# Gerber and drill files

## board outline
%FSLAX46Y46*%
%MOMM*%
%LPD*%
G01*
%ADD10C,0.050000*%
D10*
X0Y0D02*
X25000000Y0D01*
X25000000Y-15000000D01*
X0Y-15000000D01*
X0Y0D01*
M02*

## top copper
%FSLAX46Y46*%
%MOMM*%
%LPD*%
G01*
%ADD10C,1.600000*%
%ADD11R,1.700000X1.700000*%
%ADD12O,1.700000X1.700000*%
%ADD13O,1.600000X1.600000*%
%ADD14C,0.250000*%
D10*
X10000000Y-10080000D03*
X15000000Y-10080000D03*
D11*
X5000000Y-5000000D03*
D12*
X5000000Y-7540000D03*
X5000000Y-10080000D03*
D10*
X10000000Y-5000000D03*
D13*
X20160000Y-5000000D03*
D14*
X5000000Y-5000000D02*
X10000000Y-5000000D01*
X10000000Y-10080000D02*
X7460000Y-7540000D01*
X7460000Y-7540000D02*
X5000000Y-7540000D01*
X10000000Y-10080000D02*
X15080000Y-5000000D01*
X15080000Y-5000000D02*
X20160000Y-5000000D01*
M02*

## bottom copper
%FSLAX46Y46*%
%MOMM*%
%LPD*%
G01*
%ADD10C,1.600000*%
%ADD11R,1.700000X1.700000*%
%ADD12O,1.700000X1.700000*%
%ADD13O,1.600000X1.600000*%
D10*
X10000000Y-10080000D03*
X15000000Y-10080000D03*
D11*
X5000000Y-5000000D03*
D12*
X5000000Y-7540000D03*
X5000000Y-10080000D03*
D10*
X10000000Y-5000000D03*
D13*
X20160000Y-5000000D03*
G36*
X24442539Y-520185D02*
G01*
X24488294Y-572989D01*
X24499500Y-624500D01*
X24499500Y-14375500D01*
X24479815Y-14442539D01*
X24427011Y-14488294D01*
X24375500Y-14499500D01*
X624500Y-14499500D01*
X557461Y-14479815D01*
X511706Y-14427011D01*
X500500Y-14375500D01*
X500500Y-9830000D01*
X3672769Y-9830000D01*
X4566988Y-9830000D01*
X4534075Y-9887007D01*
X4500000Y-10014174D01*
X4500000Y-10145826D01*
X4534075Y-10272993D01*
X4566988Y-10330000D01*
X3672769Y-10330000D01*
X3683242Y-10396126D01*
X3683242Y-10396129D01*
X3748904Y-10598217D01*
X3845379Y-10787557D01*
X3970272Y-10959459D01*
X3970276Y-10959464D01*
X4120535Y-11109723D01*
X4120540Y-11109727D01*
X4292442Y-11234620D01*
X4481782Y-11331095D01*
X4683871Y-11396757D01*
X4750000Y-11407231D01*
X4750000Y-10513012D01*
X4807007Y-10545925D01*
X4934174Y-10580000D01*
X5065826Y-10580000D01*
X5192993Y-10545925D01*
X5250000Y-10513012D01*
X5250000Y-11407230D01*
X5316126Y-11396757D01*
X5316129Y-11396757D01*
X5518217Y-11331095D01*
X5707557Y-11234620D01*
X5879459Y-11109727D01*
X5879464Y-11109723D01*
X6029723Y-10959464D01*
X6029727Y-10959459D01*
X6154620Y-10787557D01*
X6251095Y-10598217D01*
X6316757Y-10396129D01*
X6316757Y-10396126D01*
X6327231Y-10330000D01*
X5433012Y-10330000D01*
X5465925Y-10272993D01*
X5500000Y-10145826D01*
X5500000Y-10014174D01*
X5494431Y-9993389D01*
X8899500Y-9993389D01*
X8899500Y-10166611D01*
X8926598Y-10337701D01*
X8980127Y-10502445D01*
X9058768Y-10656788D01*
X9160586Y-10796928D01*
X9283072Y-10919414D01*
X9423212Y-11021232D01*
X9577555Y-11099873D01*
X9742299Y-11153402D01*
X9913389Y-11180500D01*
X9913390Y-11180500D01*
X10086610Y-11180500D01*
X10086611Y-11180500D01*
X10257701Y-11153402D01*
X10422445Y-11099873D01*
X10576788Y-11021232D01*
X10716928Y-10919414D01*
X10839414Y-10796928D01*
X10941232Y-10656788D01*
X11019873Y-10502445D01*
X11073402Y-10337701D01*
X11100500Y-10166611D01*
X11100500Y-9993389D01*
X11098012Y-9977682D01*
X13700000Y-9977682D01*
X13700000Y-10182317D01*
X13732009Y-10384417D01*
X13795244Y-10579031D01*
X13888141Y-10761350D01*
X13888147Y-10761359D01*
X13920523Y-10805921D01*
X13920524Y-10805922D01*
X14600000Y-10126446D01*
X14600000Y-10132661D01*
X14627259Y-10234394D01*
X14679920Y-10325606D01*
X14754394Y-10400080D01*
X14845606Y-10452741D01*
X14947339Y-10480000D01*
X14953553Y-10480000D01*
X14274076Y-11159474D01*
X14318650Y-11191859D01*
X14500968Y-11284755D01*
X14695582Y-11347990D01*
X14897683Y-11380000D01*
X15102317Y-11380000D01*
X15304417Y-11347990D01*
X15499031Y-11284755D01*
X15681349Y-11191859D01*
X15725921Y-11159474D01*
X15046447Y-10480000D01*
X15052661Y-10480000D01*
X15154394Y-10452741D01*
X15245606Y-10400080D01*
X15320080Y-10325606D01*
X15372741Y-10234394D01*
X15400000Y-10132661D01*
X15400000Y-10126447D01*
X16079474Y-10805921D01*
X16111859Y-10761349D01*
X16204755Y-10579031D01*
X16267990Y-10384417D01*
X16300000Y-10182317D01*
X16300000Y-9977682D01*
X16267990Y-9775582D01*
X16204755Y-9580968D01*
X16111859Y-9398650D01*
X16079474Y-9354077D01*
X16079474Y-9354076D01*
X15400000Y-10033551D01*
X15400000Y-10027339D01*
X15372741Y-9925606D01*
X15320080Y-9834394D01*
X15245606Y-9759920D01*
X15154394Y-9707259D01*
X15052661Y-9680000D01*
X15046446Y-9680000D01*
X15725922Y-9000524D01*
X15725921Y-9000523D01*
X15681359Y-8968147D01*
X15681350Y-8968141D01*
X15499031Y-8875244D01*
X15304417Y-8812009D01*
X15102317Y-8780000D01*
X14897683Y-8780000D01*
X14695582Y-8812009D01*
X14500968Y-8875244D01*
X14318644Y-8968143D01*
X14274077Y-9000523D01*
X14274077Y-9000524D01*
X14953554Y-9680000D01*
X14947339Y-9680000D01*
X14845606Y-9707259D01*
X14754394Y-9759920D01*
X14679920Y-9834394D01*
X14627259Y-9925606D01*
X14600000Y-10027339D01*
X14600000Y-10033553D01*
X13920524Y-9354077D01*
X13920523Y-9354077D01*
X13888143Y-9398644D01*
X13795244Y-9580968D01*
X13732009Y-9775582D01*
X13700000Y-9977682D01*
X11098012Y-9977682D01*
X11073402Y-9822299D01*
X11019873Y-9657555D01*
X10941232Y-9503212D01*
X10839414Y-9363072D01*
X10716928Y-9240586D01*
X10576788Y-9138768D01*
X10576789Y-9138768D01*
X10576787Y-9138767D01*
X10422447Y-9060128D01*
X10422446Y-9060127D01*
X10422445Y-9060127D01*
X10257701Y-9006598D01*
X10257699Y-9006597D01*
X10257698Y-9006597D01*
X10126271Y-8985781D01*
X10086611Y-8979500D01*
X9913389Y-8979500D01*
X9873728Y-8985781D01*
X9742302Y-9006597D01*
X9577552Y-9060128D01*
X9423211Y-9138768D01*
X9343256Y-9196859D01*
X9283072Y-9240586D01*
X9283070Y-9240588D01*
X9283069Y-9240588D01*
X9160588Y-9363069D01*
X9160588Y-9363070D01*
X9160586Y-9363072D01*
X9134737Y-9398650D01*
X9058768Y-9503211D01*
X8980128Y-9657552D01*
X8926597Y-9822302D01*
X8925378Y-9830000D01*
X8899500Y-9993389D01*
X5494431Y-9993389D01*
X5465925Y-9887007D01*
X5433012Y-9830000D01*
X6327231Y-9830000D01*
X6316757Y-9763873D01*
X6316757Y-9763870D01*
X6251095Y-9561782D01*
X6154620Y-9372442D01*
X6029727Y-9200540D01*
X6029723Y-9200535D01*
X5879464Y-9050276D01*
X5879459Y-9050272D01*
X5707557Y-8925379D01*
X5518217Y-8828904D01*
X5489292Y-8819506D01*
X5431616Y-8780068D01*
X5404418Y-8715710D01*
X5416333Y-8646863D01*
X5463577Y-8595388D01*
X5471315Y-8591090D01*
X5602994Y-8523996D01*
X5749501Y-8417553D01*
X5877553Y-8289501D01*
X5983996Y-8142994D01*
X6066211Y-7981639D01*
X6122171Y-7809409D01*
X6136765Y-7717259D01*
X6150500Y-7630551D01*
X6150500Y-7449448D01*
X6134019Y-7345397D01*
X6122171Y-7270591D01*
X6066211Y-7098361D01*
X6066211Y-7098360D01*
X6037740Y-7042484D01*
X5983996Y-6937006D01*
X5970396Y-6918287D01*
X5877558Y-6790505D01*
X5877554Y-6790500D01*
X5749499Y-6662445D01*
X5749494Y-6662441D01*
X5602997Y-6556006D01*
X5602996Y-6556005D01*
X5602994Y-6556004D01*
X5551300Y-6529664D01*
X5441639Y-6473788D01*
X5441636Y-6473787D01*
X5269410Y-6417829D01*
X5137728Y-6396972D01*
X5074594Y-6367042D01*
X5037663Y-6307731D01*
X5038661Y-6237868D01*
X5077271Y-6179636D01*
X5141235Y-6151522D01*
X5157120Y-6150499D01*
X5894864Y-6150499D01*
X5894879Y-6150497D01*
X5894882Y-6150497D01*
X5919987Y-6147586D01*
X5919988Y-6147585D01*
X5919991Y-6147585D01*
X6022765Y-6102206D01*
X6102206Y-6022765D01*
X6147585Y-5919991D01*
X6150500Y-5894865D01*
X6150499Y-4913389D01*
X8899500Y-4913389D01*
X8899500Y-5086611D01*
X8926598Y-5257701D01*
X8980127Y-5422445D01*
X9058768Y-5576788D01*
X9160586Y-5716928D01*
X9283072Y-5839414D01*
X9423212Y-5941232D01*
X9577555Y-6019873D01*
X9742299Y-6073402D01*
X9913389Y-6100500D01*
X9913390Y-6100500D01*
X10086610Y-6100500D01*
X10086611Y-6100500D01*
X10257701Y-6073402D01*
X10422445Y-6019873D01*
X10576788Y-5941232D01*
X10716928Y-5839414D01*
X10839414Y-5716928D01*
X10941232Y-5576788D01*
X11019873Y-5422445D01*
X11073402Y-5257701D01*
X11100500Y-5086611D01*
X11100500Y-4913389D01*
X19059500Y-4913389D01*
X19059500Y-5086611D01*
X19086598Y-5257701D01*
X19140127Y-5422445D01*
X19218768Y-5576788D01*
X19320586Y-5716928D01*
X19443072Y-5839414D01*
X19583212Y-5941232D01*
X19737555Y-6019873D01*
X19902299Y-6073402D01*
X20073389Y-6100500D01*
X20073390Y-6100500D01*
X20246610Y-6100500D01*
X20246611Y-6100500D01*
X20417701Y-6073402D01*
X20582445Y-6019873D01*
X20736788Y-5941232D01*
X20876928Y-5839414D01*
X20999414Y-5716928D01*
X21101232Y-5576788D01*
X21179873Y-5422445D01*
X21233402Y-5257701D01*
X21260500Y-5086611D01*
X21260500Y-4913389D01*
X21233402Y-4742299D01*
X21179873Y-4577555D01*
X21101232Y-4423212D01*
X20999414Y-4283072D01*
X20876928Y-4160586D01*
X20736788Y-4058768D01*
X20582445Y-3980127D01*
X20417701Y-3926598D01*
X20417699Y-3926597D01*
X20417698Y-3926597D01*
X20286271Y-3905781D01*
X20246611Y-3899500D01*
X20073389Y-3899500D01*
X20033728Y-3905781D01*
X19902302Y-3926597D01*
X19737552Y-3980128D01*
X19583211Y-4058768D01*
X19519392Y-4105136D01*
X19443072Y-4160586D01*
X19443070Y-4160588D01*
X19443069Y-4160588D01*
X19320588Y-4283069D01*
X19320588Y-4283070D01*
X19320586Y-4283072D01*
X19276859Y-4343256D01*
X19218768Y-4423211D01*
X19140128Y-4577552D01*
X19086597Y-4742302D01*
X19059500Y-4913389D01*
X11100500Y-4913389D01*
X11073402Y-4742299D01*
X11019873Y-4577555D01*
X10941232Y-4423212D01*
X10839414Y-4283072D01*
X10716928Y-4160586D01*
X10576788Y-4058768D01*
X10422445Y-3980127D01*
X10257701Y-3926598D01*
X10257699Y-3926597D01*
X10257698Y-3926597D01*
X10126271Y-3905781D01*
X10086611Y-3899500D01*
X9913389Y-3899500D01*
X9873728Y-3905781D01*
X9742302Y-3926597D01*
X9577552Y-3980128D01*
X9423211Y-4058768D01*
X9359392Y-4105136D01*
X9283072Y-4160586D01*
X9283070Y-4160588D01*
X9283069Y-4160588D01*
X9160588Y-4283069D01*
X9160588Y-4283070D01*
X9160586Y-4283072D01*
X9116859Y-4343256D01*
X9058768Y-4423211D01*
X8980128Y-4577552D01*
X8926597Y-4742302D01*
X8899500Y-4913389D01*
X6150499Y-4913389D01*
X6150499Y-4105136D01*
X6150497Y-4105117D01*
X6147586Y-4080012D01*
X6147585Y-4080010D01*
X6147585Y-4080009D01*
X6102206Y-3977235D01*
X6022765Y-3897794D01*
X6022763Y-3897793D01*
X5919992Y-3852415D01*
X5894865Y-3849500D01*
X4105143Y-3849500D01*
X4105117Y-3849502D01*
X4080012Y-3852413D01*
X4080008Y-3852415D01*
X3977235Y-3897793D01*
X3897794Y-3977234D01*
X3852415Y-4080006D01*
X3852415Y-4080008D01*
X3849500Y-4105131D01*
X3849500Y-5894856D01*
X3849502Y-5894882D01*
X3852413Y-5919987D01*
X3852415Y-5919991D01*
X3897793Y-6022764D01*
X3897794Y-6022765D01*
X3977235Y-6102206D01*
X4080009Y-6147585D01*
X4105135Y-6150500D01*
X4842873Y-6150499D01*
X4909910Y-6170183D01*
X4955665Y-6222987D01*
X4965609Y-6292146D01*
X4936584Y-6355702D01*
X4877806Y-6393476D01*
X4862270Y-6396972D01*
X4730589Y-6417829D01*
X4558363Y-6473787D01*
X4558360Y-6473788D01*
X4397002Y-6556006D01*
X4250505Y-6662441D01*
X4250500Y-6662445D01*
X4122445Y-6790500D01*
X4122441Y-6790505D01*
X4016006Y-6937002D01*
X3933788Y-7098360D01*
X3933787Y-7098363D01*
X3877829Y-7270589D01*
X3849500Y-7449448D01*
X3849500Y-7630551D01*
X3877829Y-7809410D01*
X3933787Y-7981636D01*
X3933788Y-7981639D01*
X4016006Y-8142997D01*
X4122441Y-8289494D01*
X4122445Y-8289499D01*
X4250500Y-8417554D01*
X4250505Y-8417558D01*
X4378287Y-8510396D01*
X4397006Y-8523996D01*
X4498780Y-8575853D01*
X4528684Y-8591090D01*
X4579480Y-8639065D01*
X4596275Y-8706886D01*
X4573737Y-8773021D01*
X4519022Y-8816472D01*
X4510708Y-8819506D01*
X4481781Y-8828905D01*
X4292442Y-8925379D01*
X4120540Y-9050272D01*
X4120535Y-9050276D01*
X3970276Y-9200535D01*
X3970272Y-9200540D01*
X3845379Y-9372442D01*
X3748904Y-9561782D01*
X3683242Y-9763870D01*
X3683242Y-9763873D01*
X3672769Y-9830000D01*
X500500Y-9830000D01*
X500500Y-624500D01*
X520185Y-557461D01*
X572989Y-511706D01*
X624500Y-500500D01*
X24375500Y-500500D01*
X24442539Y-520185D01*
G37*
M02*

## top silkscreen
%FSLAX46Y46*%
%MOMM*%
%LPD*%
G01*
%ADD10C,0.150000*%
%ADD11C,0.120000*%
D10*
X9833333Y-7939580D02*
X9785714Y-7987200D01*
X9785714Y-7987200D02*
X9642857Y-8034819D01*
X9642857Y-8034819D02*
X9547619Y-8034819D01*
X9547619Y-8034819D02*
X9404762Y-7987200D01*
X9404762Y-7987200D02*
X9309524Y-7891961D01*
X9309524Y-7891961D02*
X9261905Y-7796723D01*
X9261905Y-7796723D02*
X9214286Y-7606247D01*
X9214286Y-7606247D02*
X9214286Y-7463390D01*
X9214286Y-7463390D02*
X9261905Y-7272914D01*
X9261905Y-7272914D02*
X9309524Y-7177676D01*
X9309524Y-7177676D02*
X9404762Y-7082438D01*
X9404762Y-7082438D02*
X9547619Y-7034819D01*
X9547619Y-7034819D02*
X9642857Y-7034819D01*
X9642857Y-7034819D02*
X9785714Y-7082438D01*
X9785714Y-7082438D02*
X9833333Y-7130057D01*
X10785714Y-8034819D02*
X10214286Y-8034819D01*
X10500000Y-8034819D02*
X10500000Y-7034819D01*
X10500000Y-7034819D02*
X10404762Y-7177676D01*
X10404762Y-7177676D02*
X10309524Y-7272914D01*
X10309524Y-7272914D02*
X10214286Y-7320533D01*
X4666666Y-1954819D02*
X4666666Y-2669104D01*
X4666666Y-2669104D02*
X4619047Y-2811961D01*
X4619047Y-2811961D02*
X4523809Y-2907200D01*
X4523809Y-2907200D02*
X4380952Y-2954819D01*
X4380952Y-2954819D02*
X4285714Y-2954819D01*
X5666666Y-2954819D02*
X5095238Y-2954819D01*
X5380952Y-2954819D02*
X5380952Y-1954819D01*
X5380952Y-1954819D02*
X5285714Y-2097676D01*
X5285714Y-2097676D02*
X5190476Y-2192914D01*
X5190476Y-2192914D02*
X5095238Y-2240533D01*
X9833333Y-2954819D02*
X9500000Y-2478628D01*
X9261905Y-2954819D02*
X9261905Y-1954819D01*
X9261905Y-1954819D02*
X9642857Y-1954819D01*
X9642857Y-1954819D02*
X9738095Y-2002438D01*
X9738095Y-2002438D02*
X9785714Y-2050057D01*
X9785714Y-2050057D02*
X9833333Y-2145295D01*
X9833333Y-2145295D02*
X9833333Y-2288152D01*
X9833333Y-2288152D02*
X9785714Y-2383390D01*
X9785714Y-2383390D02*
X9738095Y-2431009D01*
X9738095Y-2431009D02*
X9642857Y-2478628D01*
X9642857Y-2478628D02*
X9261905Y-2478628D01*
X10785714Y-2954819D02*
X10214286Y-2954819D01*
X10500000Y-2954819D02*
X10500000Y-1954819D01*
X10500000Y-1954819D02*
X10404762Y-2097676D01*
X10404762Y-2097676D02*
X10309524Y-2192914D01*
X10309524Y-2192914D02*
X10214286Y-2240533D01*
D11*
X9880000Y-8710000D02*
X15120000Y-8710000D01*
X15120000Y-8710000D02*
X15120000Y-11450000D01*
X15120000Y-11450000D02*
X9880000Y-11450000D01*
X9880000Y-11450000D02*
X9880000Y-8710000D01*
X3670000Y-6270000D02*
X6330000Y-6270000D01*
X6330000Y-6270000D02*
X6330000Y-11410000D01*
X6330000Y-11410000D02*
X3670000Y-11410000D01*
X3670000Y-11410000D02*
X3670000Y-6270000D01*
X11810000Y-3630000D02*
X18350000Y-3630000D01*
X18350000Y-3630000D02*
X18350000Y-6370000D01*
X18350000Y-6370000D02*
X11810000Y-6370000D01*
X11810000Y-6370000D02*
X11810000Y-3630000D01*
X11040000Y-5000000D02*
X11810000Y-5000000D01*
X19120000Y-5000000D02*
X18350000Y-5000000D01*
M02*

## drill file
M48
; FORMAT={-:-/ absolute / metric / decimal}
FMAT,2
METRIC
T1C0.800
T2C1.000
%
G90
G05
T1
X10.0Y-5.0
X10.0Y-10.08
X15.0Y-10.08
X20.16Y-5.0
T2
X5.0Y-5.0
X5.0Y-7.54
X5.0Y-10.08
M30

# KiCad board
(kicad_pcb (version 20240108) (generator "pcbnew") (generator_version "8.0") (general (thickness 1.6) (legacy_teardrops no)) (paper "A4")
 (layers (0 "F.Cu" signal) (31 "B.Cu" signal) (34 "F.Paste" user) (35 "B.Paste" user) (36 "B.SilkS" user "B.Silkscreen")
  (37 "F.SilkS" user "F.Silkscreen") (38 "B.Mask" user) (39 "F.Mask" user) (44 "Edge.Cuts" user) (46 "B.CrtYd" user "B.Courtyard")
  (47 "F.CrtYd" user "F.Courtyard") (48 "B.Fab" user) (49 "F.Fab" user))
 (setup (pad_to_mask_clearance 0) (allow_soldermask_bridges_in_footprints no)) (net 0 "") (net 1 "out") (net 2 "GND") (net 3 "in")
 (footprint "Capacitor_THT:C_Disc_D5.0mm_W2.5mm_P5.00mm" (layer "F.Cu") (at 10 10.08 0)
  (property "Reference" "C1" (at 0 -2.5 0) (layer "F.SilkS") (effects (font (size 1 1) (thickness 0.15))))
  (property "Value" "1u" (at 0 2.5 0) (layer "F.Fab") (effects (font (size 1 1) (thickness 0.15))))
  (fp_line (start -0.12 -1.37) (end 5.12 -1.37) (stroke (width 0.12) (type solid)) (layer "F.SilkS"))
  (fp_line (start 5.12 -1.37) (end 5.12 1.37) (stroke (width 0.12) (type solid)) (layer "F.SilkS"))
  (fp_line (start 5.12 1.37) (end -0.12 1.37) (stroke (width 0.12) (type solid)) (layer "F.SilkS"))
  (fp_line (start -0.12 1.37) (end -0.12 -1.37) (stroke (width 0.12) (type solid)) (layer "F.SilkS"))
  (pad "1" thru_hole circle (at 0 0 0) (size 1.6 1.6) (drill 0.8) (layers "*.Cu" "*.Mask") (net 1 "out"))
  (pad "2" thru_hole circle (at 5 0 0) (size 1.6 1.6) (drill 0.8) (layers "*.Cu" "*.Mask") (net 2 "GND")))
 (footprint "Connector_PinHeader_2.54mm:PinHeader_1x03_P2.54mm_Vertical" (layer "F.Cu") (at 5 5 0)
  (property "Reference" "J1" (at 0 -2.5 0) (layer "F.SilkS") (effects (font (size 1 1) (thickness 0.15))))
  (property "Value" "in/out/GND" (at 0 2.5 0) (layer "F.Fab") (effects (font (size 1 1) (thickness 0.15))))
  (fp_line (start -1.33 1.27) (end 1.33 1.27) (stroke (width 0.12) (type solid)) (layer "F.SilkS"))
  (fp_line (start 1.33 1.27) (end 1.33 6.41) (stroke (width 0.12) (type solid)) (layer "F.SilkS"))
  (fp_line (start 1.33 6.41) (end -1.33 6.41) (stroke (width 0.12) (type solid)) (layer "F.SilkS"))
  (fp_line (start -1.33 6.41) (end -1.33 1.27) (stroke (width 0.12) (type solid)) (layer "F.SilkS"))
  (pad "1" thru_hole rect (at 0 0 0) (size 1.7 1.7) (drill 1) (layers "*.Cu" "*.Mask") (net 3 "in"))
  (pad "2" thru_hole oval (at 0 2.54 0) (size 1.7 1.7) (drill 1) (layers "*.Cu" "*.Mask") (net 1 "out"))
  (pad "3" thru_hole oval (at 0 5.08 0) (size 1.7 1.7) (drill 1) (layers "*.Cu" "*.Mask") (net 2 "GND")))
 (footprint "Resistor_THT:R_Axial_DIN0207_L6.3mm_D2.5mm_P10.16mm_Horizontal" (layer "F.Cu") (at 10 5 0)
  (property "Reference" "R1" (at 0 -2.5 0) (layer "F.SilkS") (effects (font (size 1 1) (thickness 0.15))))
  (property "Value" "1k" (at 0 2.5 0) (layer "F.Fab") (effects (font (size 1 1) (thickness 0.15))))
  (fp_line (start 1.81 -1.37) (end 8.35 -1.37) (stroke (width 0.12) (type solid)) (layer "F.SilkS"))
  (fp_line (start 8.35 -1.37) (end 8.35 1.37) (stroke (width 0.12) (type solid)) (layer "F.SilkS"))
  (fp_line (start 8.35 1.37) (end 1.81 1.37) (stroke (width 0.12) (type solid)) (layer "F.SilkS"))
  (fp_line (start 1.81 1.37) (end 1.81 -1.37) (stroke (width 0.12) (type solid)) (layer "F.SilkS"))
  (fp_line (start 1.04 0) (end 1.81 0) (stroke (width 0.12) (type solid)) (layer "F.SilkS"))
  (fp_line (start 9.12 0) (end 8.35 0) (stroke (width 0.12) (type solid)) (layer "F.SilkS"))
  (pad "1" thru_hole circle (at 0 0 0) (size 1.6 1.6) (drill 0.8) (layers "*.Cu" "*.Mask") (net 3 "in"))
  (pad "2" thru_hole oval (at 10.16 0 0) (size 1.6 1.6) (drill 0.8) (layers "*.Cu" "*.Mask") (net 1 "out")))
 (gr_rect (start 0 0) (end 25 15) (stroke (width 0.05) (type default)) (fill none) (layer "Edge.Cuts"))
 (segment (start 5 5) (end 10 5) (width 0.25) (layer "F.Cu") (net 3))
 (segment (start 10 10.08) (end 7.46 7.54) (width 0.25) (layer "F.Cu") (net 1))
 (segment (start 7.46 7.54) (end 5 7.54) (width 0.25) (layer "F.Cu") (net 1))
 (segment (start 10 10.08) (end 15.08 5) (width 0.25) (layer "F.Cu") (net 1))
 (segment (start 15.08 5) (end 20.16 5) (width 0.25) (layer "F.Cu") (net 1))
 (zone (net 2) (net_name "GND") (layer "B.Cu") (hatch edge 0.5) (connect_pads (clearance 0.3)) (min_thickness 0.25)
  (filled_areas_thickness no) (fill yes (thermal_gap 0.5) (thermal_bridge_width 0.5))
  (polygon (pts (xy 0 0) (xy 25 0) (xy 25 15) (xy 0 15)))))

